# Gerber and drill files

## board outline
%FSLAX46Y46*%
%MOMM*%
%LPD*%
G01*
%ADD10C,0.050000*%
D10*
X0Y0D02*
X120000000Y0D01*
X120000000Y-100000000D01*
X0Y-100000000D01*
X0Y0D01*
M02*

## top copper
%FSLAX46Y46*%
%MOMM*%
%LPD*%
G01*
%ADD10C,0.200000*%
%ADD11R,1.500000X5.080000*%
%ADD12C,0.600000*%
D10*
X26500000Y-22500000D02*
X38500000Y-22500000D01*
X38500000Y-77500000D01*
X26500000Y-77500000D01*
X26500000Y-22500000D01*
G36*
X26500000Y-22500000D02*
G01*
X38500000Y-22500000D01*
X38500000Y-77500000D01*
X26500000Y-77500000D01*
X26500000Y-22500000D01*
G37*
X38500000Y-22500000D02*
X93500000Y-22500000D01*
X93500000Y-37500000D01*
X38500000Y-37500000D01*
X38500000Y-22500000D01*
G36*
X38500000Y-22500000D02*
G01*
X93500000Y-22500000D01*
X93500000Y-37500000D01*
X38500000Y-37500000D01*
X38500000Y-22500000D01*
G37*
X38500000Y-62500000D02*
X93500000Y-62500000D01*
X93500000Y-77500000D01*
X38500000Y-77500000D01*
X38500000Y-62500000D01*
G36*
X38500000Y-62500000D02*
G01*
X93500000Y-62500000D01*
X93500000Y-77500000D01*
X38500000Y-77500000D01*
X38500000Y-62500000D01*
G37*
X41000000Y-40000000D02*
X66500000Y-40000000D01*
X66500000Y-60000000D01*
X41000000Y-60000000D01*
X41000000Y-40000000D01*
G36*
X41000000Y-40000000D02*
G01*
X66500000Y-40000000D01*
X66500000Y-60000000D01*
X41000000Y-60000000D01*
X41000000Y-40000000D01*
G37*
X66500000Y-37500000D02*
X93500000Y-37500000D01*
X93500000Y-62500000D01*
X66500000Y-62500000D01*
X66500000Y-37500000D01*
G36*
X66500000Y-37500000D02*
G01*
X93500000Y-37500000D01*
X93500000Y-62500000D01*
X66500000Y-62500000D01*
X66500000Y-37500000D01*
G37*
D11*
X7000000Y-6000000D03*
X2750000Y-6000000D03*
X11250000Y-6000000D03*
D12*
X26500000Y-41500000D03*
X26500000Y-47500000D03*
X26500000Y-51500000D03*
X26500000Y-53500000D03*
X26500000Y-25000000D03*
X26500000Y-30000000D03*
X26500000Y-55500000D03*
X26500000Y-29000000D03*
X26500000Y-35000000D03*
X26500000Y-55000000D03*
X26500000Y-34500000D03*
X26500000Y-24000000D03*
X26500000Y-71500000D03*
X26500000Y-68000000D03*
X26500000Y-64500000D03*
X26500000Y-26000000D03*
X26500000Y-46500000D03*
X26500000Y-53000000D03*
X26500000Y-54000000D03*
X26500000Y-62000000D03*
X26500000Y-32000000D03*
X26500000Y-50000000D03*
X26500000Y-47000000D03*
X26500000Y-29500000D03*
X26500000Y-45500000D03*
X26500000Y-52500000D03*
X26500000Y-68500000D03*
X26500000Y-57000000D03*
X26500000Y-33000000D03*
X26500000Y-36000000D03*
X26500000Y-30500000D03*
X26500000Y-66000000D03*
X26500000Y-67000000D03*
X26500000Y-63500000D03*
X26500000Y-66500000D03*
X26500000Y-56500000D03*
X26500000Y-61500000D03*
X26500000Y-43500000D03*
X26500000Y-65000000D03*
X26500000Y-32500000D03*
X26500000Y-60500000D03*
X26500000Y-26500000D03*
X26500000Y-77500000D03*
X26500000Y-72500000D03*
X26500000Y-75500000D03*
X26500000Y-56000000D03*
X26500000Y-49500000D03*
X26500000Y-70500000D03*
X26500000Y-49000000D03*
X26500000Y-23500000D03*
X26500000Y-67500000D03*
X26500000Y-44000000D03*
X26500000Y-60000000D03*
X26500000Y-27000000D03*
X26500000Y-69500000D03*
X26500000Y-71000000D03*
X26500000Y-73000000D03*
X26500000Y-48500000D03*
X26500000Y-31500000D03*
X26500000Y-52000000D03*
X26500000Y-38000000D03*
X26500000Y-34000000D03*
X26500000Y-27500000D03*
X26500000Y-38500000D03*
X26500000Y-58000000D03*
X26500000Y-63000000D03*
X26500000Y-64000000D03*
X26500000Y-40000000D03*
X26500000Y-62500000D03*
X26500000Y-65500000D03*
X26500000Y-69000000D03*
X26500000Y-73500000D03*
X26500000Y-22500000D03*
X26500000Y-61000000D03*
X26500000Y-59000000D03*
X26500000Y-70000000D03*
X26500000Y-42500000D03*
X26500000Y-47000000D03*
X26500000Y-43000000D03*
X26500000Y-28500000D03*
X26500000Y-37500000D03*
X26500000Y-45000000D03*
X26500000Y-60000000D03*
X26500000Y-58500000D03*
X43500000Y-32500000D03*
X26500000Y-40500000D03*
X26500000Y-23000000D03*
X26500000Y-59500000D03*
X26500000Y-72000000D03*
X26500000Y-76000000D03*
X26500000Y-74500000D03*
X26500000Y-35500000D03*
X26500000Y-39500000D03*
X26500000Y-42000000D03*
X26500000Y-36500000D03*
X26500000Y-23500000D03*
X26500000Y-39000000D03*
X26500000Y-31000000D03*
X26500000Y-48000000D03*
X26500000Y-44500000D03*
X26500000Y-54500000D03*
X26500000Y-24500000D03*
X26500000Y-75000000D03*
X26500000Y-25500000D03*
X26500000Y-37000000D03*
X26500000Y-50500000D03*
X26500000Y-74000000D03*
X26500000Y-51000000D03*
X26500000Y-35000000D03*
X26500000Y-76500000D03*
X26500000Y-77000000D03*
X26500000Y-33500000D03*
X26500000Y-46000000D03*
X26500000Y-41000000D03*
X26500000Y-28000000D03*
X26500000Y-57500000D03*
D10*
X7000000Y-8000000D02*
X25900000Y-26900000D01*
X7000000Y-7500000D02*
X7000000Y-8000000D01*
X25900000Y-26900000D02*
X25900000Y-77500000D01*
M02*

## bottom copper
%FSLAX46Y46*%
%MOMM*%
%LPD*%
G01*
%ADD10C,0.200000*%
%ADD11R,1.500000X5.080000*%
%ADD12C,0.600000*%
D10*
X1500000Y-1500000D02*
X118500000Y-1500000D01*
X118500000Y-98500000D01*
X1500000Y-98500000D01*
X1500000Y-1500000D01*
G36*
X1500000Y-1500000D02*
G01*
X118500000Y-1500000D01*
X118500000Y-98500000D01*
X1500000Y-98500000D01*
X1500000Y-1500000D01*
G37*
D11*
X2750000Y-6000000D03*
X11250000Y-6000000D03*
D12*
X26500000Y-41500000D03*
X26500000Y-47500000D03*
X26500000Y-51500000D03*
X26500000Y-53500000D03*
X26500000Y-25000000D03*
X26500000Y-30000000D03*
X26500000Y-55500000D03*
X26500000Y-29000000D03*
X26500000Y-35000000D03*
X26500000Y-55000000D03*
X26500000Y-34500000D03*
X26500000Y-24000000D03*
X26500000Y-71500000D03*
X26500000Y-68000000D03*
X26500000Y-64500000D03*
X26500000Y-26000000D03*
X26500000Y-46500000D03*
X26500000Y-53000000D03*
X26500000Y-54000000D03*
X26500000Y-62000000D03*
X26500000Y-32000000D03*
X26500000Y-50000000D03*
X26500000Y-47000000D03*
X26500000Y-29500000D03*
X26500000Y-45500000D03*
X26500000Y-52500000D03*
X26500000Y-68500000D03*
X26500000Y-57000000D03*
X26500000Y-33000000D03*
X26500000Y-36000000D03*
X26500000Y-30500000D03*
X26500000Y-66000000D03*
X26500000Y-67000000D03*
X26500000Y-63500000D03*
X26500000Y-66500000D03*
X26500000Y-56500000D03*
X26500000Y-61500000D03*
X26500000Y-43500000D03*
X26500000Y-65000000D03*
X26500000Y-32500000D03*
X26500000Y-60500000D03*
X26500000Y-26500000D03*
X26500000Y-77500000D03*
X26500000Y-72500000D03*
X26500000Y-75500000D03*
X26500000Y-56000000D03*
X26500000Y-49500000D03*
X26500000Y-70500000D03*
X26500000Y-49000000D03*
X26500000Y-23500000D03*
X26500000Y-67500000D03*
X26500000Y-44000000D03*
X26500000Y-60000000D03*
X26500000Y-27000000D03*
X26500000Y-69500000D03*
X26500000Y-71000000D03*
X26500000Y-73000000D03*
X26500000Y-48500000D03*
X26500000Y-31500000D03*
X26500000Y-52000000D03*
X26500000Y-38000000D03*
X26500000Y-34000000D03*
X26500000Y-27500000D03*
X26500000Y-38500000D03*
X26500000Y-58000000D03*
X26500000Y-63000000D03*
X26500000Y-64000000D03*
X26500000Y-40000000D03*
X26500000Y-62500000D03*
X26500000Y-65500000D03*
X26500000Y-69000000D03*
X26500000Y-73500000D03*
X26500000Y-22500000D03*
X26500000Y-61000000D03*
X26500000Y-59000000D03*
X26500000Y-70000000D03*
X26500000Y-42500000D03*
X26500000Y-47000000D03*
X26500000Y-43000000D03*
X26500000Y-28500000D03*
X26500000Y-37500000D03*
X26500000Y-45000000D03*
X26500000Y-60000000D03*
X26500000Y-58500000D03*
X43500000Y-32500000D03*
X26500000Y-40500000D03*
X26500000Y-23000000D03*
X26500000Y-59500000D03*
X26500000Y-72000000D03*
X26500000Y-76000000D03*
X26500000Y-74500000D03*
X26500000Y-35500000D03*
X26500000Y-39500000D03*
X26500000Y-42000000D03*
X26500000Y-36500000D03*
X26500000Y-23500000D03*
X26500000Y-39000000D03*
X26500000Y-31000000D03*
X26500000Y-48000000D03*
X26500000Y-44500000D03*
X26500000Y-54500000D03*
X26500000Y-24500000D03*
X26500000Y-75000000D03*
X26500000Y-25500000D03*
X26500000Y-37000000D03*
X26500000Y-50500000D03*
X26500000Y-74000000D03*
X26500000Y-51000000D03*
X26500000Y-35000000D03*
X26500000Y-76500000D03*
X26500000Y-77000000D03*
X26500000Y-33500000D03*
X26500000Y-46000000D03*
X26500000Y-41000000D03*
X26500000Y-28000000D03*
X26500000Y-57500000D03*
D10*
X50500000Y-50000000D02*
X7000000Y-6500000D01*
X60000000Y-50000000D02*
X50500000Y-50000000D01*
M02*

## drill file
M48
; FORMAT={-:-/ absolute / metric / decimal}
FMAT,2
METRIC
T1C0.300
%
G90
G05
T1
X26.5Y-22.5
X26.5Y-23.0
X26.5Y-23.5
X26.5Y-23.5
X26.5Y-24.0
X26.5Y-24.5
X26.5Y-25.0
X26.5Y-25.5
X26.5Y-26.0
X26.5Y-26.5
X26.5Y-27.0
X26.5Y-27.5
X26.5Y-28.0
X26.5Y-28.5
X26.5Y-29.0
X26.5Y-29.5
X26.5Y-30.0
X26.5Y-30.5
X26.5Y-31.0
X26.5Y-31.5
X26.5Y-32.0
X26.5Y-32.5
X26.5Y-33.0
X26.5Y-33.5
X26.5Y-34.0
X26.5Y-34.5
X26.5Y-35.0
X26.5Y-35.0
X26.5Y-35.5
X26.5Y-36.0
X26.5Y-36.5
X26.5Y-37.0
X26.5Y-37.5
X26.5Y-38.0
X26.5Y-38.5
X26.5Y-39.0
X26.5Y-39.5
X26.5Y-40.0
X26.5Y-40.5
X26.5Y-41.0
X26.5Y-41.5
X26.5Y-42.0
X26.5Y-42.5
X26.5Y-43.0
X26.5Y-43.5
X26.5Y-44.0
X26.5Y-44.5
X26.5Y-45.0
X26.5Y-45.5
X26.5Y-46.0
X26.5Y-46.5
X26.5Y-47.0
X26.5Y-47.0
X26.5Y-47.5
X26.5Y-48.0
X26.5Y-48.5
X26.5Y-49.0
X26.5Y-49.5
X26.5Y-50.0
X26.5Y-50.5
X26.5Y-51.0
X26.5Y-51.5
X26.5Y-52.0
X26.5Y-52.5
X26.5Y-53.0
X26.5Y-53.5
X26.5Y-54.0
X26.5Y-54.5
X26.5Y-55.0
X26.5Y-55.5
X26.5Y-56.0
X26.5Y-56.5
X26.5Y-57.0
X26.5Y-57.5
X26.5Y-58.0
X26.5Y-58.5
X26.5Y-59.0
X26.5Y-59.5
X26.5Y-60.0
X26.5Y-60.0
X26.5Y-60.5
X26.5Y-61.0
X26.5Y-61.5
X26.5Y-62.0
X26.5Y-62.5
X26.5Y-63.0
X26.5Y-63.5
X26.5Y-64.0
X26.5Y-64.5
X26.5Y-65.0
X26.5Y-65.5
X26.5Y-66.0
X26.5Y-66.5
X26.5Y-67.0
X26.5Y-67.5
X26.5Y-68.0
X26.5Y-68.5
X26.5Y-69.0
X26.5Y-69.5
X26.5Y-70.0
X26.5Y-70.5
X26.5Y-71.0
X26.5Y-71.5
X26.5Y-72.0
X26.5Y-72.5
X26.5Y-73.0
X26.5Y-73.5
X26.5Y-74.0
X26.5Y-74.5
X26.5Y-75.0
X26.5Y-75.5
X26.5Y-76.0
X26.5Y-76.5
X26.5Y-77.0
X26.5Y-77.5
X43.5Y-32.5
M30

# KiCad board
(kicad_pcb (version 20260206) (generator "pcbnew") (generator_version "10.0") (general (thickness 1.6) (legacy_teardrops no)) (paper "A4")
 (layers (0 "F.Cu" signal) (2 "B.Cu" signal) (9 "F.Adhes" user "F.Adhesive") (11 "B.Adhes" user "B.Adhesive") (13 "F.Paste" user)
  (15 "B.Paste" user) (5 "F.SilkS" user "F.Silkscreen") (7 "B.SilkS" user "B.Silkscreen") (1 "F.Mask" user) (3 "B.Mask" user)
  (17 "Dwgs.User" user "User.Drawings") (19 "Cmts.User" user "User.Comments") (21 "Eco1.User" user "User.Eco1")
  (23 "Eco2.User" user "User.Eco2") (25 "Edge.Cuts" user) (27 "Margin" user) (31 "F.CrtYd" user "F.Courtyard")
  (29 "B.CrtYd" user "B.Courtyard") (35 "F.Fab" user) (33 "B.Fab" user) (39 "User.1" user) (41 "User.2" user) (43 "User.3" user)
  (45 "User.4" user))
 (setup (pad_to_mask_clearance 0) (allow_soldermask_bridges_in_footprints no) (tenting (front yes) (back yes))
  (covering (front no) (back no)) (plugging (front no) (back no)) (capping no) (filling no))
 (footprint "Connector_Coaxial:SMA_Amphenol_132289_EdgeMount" (layer "F.Cu") (at 7 6 90)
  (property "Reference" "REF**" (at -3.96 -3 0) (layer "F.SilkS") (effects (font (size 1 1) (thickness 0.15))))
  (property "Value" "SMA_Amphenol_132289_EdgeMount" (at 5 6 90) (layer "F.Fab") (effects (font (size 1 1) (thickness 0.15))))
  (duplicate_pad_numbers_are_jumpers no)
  (pad "1" smd rect (at 0 0 180) (size 1.5 5.08) (layers "F.Cu" "F.Mask" "F.Paste") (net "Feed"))
  (pad "2" smd rect (at 0 -4.25 180) (size 1.5 5.08) (layers "F.Cu" "F.Mask" "F.Paste"))
  (pad "2" smd rect (at 0 -4.25 180) (size 1.5 5.08) (layers "B.Cu" "B.Mask" "B.Paste") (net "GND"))
  (pad "2" smd rect (at 0 4.25 180) (size 1.5 5.08) (layers "F.Cu" "F.Mask" "F.Paste"))
  (pad "2" smd rect (at 0 4.25 180) (size 1.5 5.08) (layers "B.Cu" "B.Mask" "B.Paste") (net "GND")))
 (gr_rect (start 26.5 22.5) (end 38.5 77.5) (stroke (width 0.2) (type default)) (fill yes) (layer "F.Cu") (net "GND"))
 (gr_rect (start 38.5 22.5) (end 93.5 37.5) (stroke (width 0.2) (type default)) (fill yes) (layer "F.Cu") (net "GND"))
 (gr_rect (start 38.5 62.5) (end 93.5 77.5) (stroke (width 0.2) (type default)) (fill yes) (layer "F.Cu") (net "GND"))
 (gr_rect (start 41 40) (end 66.5 60) (stroke (width 0.2) (type default)) (fill yes) (layer "F.Cu") (net "GND"))
 (gr_rect (start 66.5 37.5) (end 93.5 62.5) (stroke (width 0.2) (type default)) (fill yes) (layer "F.Cu") (net "GND"))
 (gr_rect (start 1.5 1.5) (end 118.5 98.5) (stroke (width 0.2) (type solid)) (fill yes) (layer "B.Cu") (net "GND"))
 (gr_rect (start 0 0) (end 120 100) (stroke (width 0.05) (type default)) (fill no) (layer "Edge.Cuts"))
 (segment (start 7 8) (end 25.9 26.9) (width 0.2) (layer "F.Cu") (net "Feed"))
 (segment (start 7 7.5) (end 7 8) (width 0.2) (layer "F.Cu") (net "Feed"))
 (segment (start 25.9 26.9) (end 25.9 77.5) (width 0.2) (layer "F.Cu") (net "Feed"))
 (via (at 26.5 41.5) (size 0.6) (drill 0.3) (layers "F.Cu" "B.Cu") (free yes) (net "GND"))
 (via (at 26.5 47.5) (size 0.6) (drill 0.3) (layers "F.Cu" "B.Cu") (free yes) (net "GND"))
 (via (at 26.5 51.5) (size 0.6) (drill 0.3) (layers "F.Cu" "B.Cu") (free yes) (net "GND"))
 (via (at 26.5 53.5) (size 0.6) (drill 0.3) (layers "F.Cu" "B.Cu") (free yes) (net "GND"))
 (via (at 26.5 25) (size 0.6) (drill 0.3) (layers "F.Cu" "B.Cu") (free yes) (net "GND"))
 (via (at 26.5 30) (size 0.6) (drill 0.3) (layers "F.Cu" "B.Cu") (free yes) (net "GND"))
 (via (at 26.5 55.5) (size 0.6) (drill 0.3) (layers "F.Cu" "B.Cu") (free yes) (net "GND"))
 (via (at 26.5 29) (size 0.6) (drill 0.3) (layers "F.Cu" "B.Cu") (free yes) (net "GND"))
 (via (at 26.5 35) (size 0.6) (drill 0.3) (layers "F.Cu" "B.Cu") (free yes) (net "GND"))
 (via (at 26.5 55) (size 0.6) (drill 0.3) (layers "F.Cu" "B.Cu") (free yes) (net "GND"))
 (via (at 26.5 34.5) (size 0.6) (drill 0.3) (layers "F.Cu" "B.Cu") (free yes) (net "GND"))
 (via (at 26.5 24) (size 0.6) (drill 0.3) (layers "F.Cu" "B.Cu") (free yes) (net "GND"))
 (via (at 26.5 71.5) (size 0.6) (drill 0.3) (layers "F.Cu" "B.Cu") (free yes) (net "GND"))
 (via (at 26.5 68) (size 0.6) (drill 0.3) (layers "F.Cu" "B.Cu") (free yes) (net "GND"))
 (via (at 26.5 64.5) (size 0.6) (drill 0.3) (layers "F.Cu" "B.Cu") (free yes) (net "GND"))
 (via (at 26.5 26) (size 0.6) (drill 0.3) (layers "F.Cu" "B.Cu") (free yes) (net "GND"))
 (via (at 26.5 46.5) (size 0.6) (drill 0.3) (layers "F.Cu" "B.Cu") (free yes) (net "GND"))
 (via (at 26.5 53) (size 0.6) (drill 0.3) (layers "F.Cu" "B.Cu") (free yes) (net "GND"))
 (via (at 26.5 54) (size 0.6) (drill 0.3) (layers "F.Cu" "B.Cu") (free yes) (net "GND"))
 (via (at 26.5 62) (size 0.6) (drill 0.3) (layers "F.Cu" "B.Cu") (free yes) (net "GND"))
 (via (at 26.5 32) (size 0.6) (drill 0.3) (layers "F.Cu" "B.Cu") (free yes) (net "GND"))
 (via (at 26.5 50) (size 0.6) (drill 0.3) (layers "F.Cu" "B.Cu") (free yes) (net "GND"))
 (via (at 26.5 47) (size 0.6) (drill 0.3) (layers "F.Cu" "B.Cu") (free yes) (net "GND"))
 (via (at 26.5 29.5) (size 0.6) (drill 0.3) (layers "F.Cu" "B.Cu") (free yes) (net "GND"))
 (via (at 26.5 45.5) (size 0.6) (drill 0.3) (layers "F.Cu" "B.Cu") (free yes) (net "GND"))
 (via (at 26.5 52.5) (size 0.6) (drill 0.3) (layers "F.Cu" "B.Cu") (free yes) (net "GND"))
 (via (at 26.5 68.5) (size 0.6) (drill 0.3) (layers "F.Cu" "B.Cu") (free yes) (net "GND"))
 (via (at 26.5 57) (size 0.6) (drill 0.3) (layers "F.Cu" "B.Cu") (free yes) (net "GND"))
 (via (at 26.5 33) (size 0.6) (drill 0.3) (layers "F.Cu" "B.Cu") (free yes) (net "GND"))
 (via (at 26.5 36) (size 0.6) (drill 0.3) (layers "F.Cu" "B.Cu") (free yes) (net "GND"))
 (via (at 26.5 30.5) (size 0.6) (drill 0.3) (layers "F.Cu" "B.Cu") (free yes) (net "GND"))
 (via (at 26.5 66) (size 0.6) (drill 0.3) (layers "F.Cu" "B.Cu") (free yes) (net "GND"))
 (via (at 26.5 67) (size 0.6) (drill 0.3) (layers "F.Cu" "B.Cu") (free yes) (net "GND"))
 (via (at 26.5 63.5) (size 0.6) (drill 0.3) (layers "F.Cu" "B.Cu") (free yes) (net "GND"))
 (via (at 26.5 66.5) (size 0.6) (drill 0.3) (layers "F.Cu" "B.Cu") (free yes) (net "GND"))
 (via (at 26.5 56.5) (size 0.6) (drill 0.3) (layers "F.Cu" "B.Cu") (free yes) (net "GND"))
 (via (at 26.5 61.5) (size 0.6) (drill 0.3) (layers "F.Cu" "B.Cu") (free yes) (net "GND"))
 (via (at 26.5 43.5) (size 0.6) (drill 0.3) (layers "F.Cu" "B.Cu") (free yes) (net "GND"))
 (via (at 26.5 65) (size 0.6) (drill 0.3) (layers "F.Cu" "B.Cu") (free yes) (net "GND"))
 (via (at 26.5 32.5) (size 0.6) (drill 0.3) (layers "F.Cu" "B.Cu") (free yes) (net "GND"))
 (via (at 26.5 60.5) (size 0.6) (drill 0.3) (layers "F.Cu" "B.Cu") (free yes) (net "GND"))
 (via (at 26.5 26.5) (size 0.6) (drill 0.3) (layers "F.Cu" "B.Cu") (free yes) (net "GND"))
 (via (at 26.5 77.5) (size 0.6) (drill 0.3) (layers "F.Cu" "B.Cu") (free yes) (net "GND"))
 (via (at 26.5 72.5) (size 0.6) (drill 0.3) (layers "F.Cu" "B.Cu") (free yes) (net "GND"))
 (via (at 26.5 75.5) (size 0.6) (drill 0.3) (layers "F.Cu" "B.Cu") (free yes) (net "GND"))
 (via (at 26.5 56) (size 0.6) (drill 0.3) (layers "F.Cu" "B.Cu") (free yes) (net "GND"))
 (via (at 26.5 49.5) (size 0.6) (drill 0.3) (layers "F.Cu" "B.Cu") (free yes) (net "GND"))
 (via (at 26.5 70.5) (size 0.6) (drill 0.3) (layers "F.Cu" "B.Cu") (free yes) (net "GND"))
 (via (at 26.5 49) (size 0.6) (drill 0.3) (layers "F.Cu" "B.Cu") (free yes) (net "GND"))
 (via (at 26.5 23.5) (size 0.6) (drill 0.3) (layers "F.Cu" "B.Cu") (free yes) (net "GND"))
 (via (at 26.5 67.5) (size 0.6) (drill 0.3) (layers "F.Cu" "B.Cu") (free yes) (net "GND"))
 (via (at 26.5 44) (size 0.6) (drill 0.3) (layers "F.Cu" "B.Cu") (free yes) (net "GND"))
 (via (at 26.5 60) (size 0.6) (drill 0.3) (layers "F.Cu" "B.Cu") (free yes) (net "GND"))
 (via (at 26.5 27) (size 0.6) (drill 0.3) (layers "F.Cu" "B.Cu") (free yes) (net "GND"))
 (via (at 26.5 69.5) (size 0.6) (drill 0.3) (layers "F.Cu" "B.Cu") (free yes) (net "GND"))
 (via (at 26.5 71) (size 0.6) (drill 0.3) (layers "F.Cu" "B.Cu") (free yes) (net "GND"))
 (via (at 26.5 73) (size 0.6) (drill 0.3) (layers "F.Cu" "B.Cu") (free yes) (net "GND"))
 (via (at 26.5 48.5) (size 0.6) (drill 0.3) (layers "F.Cu" "B.Cu") (free yes) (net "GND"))
 (via (at 26.5 31.5) (size 0.6) (drill 0.3) (layers "F.Cu" "B.Cu") (free yes) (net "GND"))
 (via (at 26.5 52) (size 0.6) (drill 0.3) (layers "F.Cu" "B.Cu") (free yes) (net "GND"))
 (via (at 26.5 38) (size 0.6) (drill 0.3) (layers "F.Cu" "B.Cu") (free yes) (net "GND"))
 (via (at 26.5 34) (size 0.6) (drill 0.3) (layers "F.Cu" "B.Cu") (free yes) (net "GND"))
 (via (at 26.5 27.5) (size 0.6) (drill 0.3) (layers "F.Cu" "B.Cu") (free yes) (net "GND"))
 (via (at 26.5 38.5) (size 0.6) (drill 0.3) (layers "F.Cu" "B.Cu") (free yes) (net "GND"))
 (via (at 26.5 58) (size 0.6) (drill 0.3) (layers "F.Cu" "B.Cu") (free yes) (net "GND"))
 (via (at 26.5 63) (size 0.6) (drill 0.3) (layers "F.Cu" "B.Cu") (free yes) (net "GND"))
 (via (at 26.5 64) (size 0.6) (drill 0.3) (layers "F.Cu" "B.Cu") (free yes) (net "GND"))
 (via (at 26.5 40) (size 0.6) (drill 0.3) (layers "F.Cu" "B.Cu") (free yes) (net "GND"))
 (via (at 26.5 62.5) (size 0.6) (drill 0.3) (layers "F.Cu" "B.Cu") (free yes) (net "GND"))
 (via (at 26.5 65.5) (size 0.6) (drill 0.3) (layers "F.Cu" "B.Cu") (free yes) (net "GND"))
 (via (at 26.5 69) (size 0.6) (drill 0.3) (layers "F.Cu" "B.Cu") (free yes) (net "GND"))
 (via (at 26.5 73.5) (size 0.6) (drill 0.3) (layers "F.Cu" "B.Cu") (free yes) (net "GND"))
 (via (at 26.5 22.5) (size 0.6) (drill 0.3) (layers "F.Cu" "B.Cu") (free yes) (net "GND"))
 (via (at 26.5 61) (size 0.6) (drill 0.3) (layers "F.Cu" "B.Cu") (free yes) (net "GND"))
 (via (at 26.5 59) (size 0.6) (drill 0.3) (layers "F.Cu" "B.Cu") (free yes) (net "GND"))
 (via (at 26.5 70) (size 0.6) (drill 0.3) (layers "F.Cu" "B.Cu") (free yes) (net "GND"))
 (via (at 26.5 42.5) (size 0.6) (drill 0.3) (layers "F.Cu" "B.Cu") (free yes) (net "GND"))
 (via (at 26.5 47) (size 0.6) (drill 0.3) (layers "F.Cu" "B.Cu") (free yes) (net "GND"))
 (via (at 26.5 43) (size 0.6) (drill 0.3) (layers "F.Cu" "B.Cu") (free yes) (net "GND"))
 (via (at 26.5 28.5) (size 0.6) (drill 0.3) (layers "F.Cu" "B.Cu") (free yes) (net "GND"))
 (via (at 26.5 37.5) (size 0.6) (drill 0.3) (layers "F.Cu" "B.Cu") (free yes) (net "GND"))
 (via (at 26.5 45) (size 0.6) (drill 0.3) (layers "F.Cu" "B.Cu") (free yes) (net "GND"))
 (via (at 26.5 60) (size 0.6) (drill 0.3) (layers "F.Cu" "B.Cu") (free yes) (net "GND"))
 (via (at 26.5 58.5) (size 0.6) (drill 0.3) (layers "F.Cu" "B.Cu") (free yes) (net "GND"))
 (via (at 43.5 32.5) (size 0.6) (drill 0.3) (layers "F.Cu" "B.Cu") (free yes) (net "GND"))
 (via (at 26.5 40.5) (size 0.6) (drill 0.3) (layers "F.Cu" "B.Cu") (free yes) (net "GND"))
 (via (at 26.5 23) (size 0.6) (drill 0.3) (layers "F.Cu" "B.Cu") (free yes) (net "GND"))
 (via (at 26.5 59.5) (size 0.6) (drill 0.3) (layers "F.Cu" "B.Cu") (free yes) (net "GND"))
 (via (at 26.5 72) (size 0.6) (drill 0.3) (layers "F.Cu" "B.Cu") (free yes) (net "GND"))
 (via (at 26.5 76) (size 0.6) (drill 0.3) (layers "F.Cu" "B.Cu") (free yes) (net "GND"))
 (via (at 26.5 74.5) (size 0.6) (drill 0.3) (layers "F.Cu" "B.Cu") (free yes) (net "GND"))
 (via (at 26.5 35.5) (size 0.6) (drill 0.3) (layers "F.Cu" "B.Cu") (free yes) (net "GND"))
 (via (at 26.5 39.5) (size 0.6) (drill 0.3) (layers "F.Cu" "B.Cu") (free yes) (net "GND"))
 (via (at 26.5 42) (size 0.6) (drill 0.3) (layers "F.Cu" "B.Cu") (free yes) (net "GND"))
 (via (at 26.5 36.5) (size 0.6) (drill 0.3) (layers "F.Cu" "B.Cu") (free yes) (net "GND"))
 (via (at 26.5 23.5) (size 0.6) (drill 0.3) (layers "F.Cu" "B.Cu") (free yes) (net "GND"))
 (via (at 26.5 39) (size 0.6) (drill 0.3) (layers "F.Cu" "B.Cu") (free yes) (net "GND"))
 (via (at 26.5 31) (size 0.6) (drill 0.3) (layers "F.Cu" "B.Cu") (free yes) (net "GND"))
 (via (at 26.5 48) (size 0.6) (drill 0.3) (layers "F.Cu" "B.Cu") (free yes) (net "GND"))
 (via (at 26.5 44.5) (size 0.6) (drill 0.3) (layers "F.Cu" "B.Cu") (free yes) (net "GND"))
 (via (at 26.5 54.5) (size 0.6) (drill 0.3) (layers "F.Cu" "B.Cu") (free yes) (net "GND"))
 (via (at 26.5 24.5) (size 0.6) (drill 0.3) (layers "F.Cu" "B.Cu") (free yes) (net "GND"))
 (via (at 26.5 75) (size 0.6) (drill 0.3) (layers "F.Cu" "B.Cu") (free yes) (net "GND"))
 (via (at 26.5 25.5) (size 0.6) (drill 0.3) (layers "F.Cu" "B.Cu") (free yes) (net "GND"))
 (via (at 26.5 37) (size 0.6) (drill 0.3) (layers "F.Cu" "B.Cu") (free yes) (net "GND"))
 (via (at 26.5 50.5) (size 0.6) (drill 0.3) (layers "F.Cu" "B.Cu") (free yes) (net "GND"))
 (via (at 26.5 74) (size 0.6) (drill 0.3) (layers "F.Cu" "B.Cu") (free yes) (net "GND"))
 (via (at 26.5 51) (size 0.6) (drill 0.3) (layers "F.Cu" "B.Cu") (free yes) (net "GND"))
 (via (at 26.5 35) (size 0.6) (drill 0.3) (layers "F.Cu" "B.Cu") (free yes) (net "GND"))
 (via (at 26.5 76.5) (size 0.6) (drill 0.3) (layers "F.Cu" "B.Cu") (free yes) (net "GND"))
 (via (at 26.5 77) (size 0.6) (drill 0.3) (layers "F.Cu" "B.Cu") (free yes) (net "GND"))
 (via (at 26.5 33.5) (size 0.6) (drill 0.3) (layers "F.Cu" "B.Cu") (free yes) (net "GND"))
 (via (at 26.5 46) (size 0.6) (drill 0.3) (layers "F.Cu" "B.Cu") (free yes) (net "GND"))
 (via (at 26.5 41) (size 0.6) (drill 0.3) (layers "F.Cu" "B.Cu") (free yes) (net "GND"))
 (via (at 26.5 28) (size 0.6) (drill 0.3) (layers "F.Cu" "B.Cu") (free yes) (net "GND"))
 (via (at 26.5 57.5) (size 0.6) (drill 0.3) (layers "F.Cu" "B.Cu") (free yes) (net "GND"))
 (segment (start 50.5 50) (end 7 6.5) (width 0.2) (layer "B.Cu") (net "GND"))
 (segment (start 60 50) (end 50.5 50) (width 0.2) (layer "B.Cu") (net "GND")))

